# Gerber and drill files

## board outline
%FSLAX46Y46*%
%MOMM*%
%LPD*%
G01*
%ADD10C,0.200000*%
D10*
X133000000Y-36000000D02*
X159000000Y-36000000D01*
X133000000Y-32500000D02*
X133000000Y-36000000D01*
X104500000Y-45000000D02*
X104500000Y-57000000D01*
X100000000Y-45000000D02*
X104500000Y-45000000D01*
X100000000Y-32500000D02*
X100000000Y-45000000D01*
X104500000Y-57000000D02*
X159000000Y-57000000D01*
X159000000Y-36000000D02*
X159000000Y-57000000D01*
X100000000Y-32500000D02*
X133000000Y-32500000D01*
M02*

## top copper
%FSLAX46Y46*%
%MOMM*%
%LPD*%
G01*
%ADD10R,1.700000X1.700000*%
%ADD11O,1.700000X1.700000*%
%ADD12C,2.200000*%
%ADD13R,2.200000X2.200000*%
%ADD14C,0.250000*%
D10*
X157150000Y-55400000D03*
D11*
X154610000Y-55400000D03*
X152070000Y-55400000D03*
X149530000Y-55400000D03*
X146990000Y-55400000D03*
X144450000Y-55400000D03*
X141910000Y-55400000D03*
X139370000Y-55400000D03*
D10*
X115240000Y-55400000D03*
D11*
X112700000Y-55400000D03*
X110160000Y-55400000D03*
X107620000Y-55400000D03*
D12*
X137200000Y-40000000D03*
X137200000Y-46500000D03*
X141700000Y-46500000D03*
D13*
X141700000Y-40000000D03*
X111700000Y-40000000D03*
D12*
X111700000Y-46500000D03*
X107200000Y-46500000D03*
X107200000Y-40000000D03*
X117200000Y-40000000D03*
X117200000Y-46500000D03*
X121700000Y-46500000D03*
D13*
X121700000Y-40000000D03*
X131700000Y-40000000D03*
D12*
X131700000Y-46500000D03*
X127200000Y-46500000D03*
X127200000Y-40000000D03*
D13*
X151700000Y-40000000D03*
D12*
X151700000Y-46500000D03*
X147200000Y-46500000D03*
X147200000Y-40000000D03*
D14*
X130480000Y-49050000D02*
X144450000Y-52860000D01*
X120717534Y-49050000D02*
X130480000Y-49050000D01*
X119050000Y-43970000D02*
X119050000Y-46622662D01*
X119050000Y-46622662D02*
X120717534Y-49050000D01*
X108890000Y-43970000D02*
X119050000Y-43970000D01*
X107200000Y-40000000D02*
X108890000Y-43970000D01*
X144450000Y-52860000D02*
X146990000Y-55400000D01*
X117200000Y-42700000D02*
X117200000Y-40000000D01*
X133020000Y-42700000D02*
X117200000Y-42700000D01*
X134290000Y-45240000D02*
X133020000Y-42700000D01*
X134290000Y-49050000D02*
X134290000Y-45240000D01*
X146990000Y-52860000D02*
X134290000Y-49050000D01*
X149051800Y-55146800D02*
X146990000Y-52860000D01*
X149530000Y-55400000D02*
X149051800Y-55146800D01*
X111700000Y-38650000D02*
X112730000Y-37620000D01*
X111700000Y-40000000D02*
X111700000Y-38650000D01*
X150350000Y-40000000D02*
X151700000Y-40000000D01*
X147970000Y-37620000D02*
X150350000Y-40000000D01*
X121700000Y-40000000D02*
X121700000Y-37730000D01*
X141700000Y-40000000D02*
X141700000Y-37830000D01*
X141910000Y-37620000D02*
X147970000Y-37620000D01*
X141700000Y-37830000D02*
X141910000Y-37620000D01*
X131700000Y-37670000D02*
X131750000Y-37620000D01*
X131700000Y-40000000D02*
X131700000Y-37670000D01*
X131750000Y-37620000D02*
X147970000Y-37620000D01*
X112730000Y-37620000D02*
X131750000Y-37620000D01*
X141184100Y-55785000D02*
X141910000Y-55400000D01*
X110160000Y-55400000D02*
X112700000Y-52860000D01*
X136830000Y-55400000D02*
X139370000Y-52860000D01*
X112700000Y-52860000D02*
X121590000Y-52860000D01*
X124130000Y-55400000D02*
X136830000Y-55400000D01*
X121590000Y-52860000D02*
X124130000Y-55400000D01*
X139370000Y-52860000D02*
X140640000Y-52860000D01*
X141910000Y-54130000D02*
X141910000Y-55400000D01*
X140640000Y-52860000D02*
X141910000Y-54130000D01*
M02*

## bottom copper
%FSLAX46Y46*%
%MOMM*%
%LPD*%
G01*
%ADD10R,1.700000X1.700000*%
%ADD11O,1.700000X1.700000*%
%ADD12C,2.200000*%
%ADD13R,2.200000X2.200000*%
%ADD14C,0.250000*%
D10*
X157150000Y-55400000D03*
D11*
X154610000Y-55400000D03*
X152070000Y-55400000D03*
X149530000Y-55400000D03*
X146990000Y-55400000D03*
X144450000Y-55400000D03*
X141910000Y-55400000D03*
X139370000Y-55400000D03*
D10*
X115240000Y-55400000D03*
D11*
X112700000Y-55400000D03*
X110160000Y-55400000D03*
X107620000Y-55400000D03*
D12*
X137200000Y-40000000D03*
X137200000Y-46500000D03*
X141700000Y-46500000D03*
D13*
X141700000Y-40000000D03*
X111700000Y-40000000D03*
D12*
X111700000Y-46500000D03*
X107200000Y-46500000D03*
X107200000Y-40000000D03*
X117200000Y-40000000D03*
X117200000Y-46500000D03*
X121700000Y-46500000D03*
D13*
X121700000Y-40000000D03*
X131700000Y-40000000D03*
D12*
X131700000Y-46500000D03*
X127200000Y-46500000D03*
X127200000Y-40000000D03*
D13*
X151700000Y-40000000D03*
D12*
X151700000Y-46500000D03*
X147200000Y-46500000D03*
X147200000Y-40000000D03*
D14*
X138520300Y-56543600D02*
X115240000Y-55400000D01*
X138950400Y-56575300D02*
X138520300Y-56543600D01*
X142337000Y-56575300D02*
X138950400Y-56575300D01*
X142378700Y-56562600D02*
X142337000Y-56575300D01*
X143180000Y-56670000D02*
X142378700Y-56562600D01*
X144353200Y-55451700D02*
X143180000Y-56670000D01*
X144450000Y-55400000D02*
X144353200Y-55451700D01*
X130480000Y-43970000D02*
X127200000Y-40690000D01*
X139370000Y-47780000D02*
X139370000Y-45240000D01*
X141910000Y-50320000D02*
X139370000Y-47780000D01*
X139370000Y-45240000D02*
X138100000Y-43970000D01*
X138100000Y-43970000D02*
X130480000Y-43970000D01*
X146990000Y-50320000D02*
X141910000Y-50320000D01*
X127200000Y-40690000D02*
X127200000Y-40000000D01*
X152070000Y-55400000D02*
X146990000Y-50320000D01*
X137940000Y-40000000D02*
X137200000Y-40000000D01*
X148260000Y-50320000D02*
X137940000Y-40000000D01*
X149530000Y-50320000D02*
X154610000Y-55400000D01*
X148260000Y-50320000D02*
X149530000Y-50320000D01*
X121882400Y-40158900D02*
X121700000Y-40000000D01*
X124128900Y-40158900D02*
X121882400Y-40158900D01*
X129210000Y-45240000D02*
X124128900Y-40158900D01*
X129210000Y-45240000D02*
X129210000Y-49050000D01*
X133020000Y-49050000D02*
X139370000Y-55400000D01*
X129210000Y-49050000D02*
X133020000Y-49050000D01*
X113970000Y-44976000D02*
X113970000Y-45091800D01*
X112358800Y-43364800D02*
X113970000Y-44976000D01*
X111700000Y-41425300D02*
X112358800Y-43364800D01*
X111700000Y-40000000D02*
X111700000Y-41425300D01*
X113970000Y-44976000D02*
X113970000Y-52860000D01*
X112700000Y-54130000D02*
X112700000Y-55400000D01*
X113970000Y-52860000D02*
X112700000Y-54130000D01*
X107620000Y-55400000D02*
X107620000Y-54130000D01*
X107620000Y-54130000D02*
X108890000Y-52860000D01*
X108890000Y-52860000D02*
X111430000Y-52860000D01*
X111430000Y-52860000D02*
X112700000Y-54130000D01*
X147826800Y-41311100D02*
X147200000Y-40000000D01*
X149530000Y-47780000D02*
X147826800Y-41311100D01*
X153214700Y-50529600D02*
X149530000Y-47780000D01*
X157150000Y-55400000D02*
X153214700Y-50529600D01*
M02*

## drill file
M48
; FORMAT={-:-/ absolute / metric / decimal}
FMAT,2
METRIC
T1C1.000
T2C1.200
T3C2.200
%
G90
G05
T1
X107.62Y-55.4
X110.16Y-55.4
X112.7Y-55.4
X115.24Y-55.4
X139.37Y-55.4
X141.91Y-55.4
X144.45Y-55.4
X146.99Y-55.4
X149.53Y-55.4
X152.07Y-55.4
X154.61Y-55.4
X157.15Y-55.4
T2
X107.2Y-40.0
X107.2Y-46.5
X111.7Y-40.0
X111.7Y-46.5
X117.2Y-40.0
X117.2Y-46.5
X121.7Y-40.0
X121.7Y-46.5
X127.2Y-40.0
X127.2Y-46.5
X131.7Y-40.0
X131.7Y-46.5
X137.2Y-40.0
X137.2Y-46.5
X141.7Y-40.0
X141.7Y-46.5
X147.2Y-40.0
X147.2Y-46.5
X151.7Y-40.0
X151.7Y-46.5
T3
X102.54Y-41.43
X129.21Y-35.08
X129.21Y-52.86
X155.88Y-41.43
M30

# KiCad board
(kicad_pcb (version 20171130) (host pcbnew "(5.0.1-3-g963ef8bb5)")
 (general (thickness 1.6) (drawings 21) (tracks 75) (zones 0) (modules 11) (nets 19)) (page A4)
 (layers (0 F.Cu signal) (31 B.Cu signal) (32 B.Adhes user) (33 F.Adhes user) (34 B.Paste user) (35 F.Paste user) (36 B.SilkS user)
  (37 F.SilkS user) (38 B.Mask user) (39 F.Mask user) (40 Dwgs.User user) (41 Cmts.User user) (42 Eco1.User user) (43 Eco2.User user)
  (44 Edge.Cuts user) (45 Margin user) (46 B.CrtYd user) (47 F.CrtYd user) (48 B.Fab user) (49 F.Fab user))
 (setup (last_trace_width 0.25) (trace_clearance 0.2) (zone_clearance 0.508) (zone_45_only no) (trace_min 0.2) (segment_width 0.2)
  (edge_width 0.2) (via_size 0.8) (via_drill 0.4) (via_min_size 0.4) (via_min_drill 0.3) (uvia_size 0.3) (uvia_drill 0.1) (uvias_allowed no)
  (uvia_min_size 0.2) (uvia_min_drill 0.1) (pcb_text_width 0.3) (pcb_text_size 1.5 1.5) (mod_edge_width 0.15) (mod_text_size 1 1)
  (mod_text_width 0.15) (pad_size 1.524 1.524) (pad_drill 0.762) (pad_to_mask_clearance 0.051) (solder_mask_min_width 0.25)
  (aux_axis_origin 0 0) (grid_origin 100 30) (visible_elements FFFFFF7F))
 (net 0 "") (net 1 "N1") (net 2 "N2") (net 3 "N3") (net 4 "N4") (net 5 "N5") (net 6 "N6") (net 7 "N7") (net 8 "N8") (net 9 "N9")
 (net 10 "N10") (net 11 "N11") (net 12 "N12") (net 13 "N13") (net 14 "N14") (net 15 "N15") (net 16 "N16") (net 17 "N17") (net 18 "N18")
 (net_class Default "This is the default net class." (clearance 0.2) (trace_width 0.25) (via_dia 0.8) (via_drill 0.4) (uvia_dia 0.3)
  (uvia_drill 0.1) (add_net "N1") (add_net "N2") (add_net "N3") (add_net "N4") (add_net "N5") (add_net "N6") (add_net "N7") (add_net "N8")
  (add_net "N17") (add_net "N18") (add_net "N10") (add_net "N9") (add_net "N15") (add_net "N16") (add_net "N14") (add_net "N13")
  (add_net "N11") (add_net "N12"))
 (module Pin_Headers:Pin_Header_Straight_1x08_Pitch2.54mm (layer F.Cu) (at 157.15 55.4 270)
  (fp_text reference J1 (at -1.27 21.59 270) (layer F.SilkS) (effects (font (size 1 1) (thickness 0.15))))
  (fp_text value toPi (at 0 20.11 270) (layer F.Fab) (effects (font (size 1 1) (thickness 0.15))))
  (pad 1 thru_hole rect (at 0 0 270) (size 1.7 1.7) (drill 1) (layers *.Cu *.Mask) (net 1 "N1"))
  (pad 2 thru_hole oval (at 0 2.54 270) (size 1.7 1.7) (drill 1) (layers *.Cu *.Mask) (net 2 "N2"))
  (pad 3 thru_hole oval (at 0 5.08 270) (size 1.7 1.7) (drill 1) (layers *.Cu *.Mask) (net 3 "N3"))
  (pad 4 thru_hole oval (at 0 7.62 270) (size 1.7 1.7) (drill 1) (layers *.Cu *.Mask) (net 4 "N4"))
  (pad 5 thru_hole oval (at 0 10.16 270) (size 1.7 1.7) (drill 1) (layers *.Cu *.Mask) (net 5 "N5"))
  (pad 6 thru_hole oval (at 0 12.7 270) (size 1.7 1.7) (drill 1) (layers *.Cu *.Mask) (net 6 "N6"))
  (pad 7 thru_hole oval (at 0 15.24 270) (size 1.7 1.7) (drill 1) (layers *.Cu *.Mask) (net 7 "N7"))
  (pad 8 thru_hole oval (at 0 17.78 270) (size 1.7 1.7) (drill 1) (layers *.Cu *.Mask) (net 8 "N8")))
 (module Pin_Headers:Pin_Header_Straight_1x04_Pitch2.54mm (layer F.Cu) (at 115.24 55.4 270)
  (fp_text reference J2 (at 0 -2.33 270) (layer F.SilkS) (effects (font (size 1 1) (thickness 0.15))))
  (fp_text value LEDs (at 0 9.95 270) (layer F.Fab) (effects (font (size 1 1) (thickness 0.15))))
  (pad 1 thru_hole rect (at 0 0 270) (size 1.7 1.7) (drill 1) (layers *.Cu *.Mask) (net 6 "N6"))
  (pad 2 thru_hole oval (at 0 2.54 270) (size 1.7 1.7) (drill 1) (layers *.Cu *.Mask) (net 8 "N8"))
  (pad 3 thru_hole oval (at 0 5.08 270) (size 1.7 1.7) (drill 1) (layers *.Cu *.Mask) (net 7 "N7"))
  (pad 4 thru_hole oval (at 0 7.62 270) (size 1.7 1.7) (drill 1) (layers *.Cu *.Mask) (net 8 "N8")))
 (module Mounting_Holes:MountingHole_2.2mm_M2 (layer F.Cu) (at 155.88 41.43)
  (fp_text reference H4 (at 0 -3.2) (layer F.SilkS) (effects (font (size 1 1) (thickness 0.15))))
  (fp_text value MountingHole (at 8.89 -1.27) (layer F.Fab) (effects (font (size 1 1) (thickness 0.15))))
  (pad 1 np_thru_hole circle (at 0 0) (size 2.2 2.2) (drill 2.2) (layers *.Cu *.Mask)))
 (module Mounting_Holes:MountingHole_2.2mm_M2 (layer F.Cu) (at 129.21 35.08)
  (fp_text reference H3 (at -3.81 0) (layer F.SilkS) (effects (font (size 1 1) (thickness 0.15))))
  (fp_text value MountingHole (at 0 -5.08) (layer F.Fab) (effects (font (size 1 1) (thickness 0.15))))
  (pad 1 np_thru_hole circle (at 0 0) (size 2.2 2.2) (drill 2.2) (layers *.Cu *.Mask)))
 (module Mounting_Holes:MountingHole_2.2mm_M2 (layer F.Cu) (at 102.54 41.43)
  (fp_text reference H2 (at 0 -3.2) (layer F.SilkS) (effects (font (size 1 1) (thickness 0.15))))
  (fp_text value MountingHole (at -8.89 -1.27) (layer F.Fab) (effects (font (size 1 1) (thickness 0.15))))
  (pad 1 np_thru_hole circle (at 0 0) (size 2.2 2.2) (drill 2.2) (layers *.Cu *.Mask)))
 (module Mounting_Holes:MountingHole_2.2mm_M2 (layer F.Cu) (at 129.21 52.86)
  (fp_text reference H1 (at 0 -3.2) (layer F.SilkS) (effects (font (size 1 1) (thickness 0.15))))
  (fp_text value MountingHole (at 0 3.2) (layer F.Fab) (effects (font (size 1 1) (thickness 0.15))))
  (pad 1 np_thru_hole circle (at 0 0) (size 2.2 2.2) (drill 2.2) (layers *.Cu *.Mask)))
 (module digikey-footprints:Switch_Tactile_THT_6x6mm (layer F.Cu) (at 141.7 40 270)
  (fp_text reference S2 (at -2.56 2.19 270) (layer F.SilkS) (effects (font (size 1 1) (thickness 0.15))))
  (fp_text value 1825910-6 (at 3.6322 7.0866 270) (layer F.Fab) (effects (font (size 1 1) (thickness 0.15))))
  (pad 3 thru_hole circle (at 0 4.5 270) (size 2.2 2.2) (drill 1.2) (layers *.Cu *.Mask) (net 2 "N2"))
  (pad 4 thru_hole circle (at 6.5 4.5 270) (size 2.2 2.2) (drill 1.2) (layers *.Cu *.Mask) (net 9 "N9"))
  (pad 2 thru_hole circle (at 6.5 0 270) (size 2.2 2.2) (drill 1.2) (layers *.Cu *.Mask) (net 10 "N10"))
  (pad 1 thru_hole rect (at 0 0 270) (size 2.2 2.2) (drill 1.2) (layers *.Cu *.Mask) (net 8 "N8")))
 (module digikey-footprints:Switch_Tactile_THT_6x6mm (layer F.Cu) (at 111.7 40 270)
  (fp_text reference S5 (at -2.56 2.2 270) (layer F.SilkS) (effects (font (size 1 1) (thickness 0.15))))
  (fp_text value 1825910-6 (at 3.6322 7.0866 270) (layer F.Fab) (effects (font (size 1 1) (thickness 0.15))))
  (pad 1 thru_hole rect (at 0 0 270) (size 2.2 2.2) (drill 1.2) (layers *.Cu *.Mask) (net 8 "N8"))
  (pad 2 thru_hole circle (at 6.5 0 270) (size 2.2 2.2) (drill 1.2) (layers *.Cu *.Mask) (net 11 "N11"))
  (pad 4 thru_hole circle (at 6.5 4.5 270) (size 2.2 2.2) (drill 1.2) (layers *.Cu *.Mask) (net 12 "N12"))
  (pad 3 thru_hole circle (at 0 4.5 270) (size 2.2 2.2) (drill 1.2) (layers *.Cu *.Mask) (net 5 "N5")))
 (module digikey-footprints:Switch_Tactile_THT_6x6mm (layer F.Cu) (at 121.7 40 270)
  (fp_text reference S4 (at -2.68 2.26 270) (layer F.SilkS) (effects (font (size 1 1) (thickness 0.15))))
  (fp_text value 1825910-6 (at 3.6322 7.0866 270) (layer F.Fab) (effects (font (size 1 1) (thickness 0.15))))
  (pad 3 thru_hole circle (at 0 4.5 270) (size 2.2 2.2) (drill 1.2) (layers *.Cu *.Mask) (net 4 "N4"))
  (pad 4 thru_hole circle (at 6.5 4.5 270) (size 2.2 2.2) (drill 1.2) (layers *.Cu *.Mask) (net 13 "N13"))
  (pad 2 thru_hole circle (at 6.5 0 270) (size 2.2 2.2) (drill 1.2) (layers *.Cu *.Mask) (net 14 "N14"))
  (pad 1 thru_hole rect (at 0 0 270) (size 2.2 2.2) (drill 1.2) (layers *.Cu *.Mask) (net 8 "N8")))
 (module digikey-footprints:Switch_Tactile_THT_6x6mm (layer F.Cu) (at 131.7 40 270)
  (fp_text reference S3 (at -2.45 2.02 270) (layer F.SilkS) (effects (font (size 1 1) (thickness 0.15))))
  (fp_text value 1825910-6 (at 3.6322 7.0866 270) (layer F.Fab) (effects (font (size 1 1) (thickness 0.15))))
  (pad 1 thru_hole rect (at 0 0 270) (size 2.2 2.2) (drill 1.2) (layers *.Cu *.Mask) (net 8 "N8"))
  (pad 2 thru_hole circle (at 6.5 0 270) (size 2.2 2.2) (drill 1.2) (layers *.Cu *.Mask) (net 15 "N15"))
  (pad 4 thru_hole circle (at 6.5 4.5 270) (size 2.2 2.2) (drill 1.2) (layers *.Cu *.Mask) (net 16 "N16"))
  (pad 3 thru_hole circle (at 0 4.5 270) (size 2.2 2.2) (drill 1.2) (layers *.Cu *.Mask) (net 3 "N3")))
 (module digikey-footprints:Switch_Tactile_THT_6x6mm (layer F.Cu) (at 151.7 40 270)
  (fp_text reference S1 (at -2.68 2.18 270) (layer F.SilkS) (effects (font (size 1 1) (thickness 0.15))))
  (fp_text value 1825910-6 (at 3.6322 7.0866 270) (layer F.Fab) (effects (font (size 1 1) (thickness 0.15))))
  (pad 1 thru_hole rect (at 0 0 270) (size 2.2 2.2) (drill 1.2) (layers *.Cu *.Mask) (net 8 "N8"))
  (pad 2 thru_hole circle (at 6.5 0 270) (size 2.2 2.2) (drill 1.2) (layers *.Cu *.Mask) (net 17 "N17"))
  (pad 4 thru_hole circle (at 6.5 4.5 270) (size 2.2 2.2) (drill 1.2) (layers *.Cu *.Mask) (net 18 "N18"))
  (pad 3 thru_hole circle (at 0 4.5 270) (size 2.2 2.2) (drill 1.2) (layers *.Cu *.Mask) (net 1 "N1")))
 (gr_line (start 133 36) (end 159 36) (layer Edge.Cuts) (width 0.2))
 (gr_line (start 133 32.5) (end 133 36) (layer Edge.Cuts) (width 0.2))
 (gr_line (start 104.5 45) (end 104.5 57) (layer Edge.Cuts) (width 0.2))
 (gr_line (start 100 45) (end 104.5 45) (layer Edge.Cuts) (width 0.2))
 (gr_line (start 100 32.5) (end 100 45) (layer Edge.Cuts) (width 0.2))
 (gr_line (start 104.5 57) (end 159 57) (layer Edge.Cuts) (width 0.2))
 (gr_line (start 159 36) (end 159 57) (layer Edge.Cuts) (width 0.2))
 (gr_line (start 100 32.5) (end 133 32.5) (layer Edge.Cuts) (width 0.2))
 (segment (start 138.5203 56.5436) (end 115.24 55.4) (width 0.25) (layer B.Cu) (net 6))
 (segment (start 138.9504 56.5753) (end 138.5203 56.5436) (width 0.25) (layer B.Cu) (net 6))
 (segment (start 142.337 56.5753) (end 138.9504 56.5753) (width 0.25) (layer B.Cu) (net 6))
 (segment (start 142.3787 56.5626) (end 142.337 56.5753) (width 0.25) (layer B.Cu) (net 6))
 (segment (start 143.18 56.67) (end 142.3787 56.5626) (width 0.25) (layer B.Cu) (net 6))
 (segment (start 144.3532 55.4517) (end 143.18 56.67) (width 0.25) (layer B.Cu) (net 6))
 (segment (start 144.45 55.4) (end 144.3532 55.4517) (width 0.25) (layer B.Cu) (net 6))
 (segment (start 130.48 49.05) (end 144.45 52.86) (width 0.25) (layer F.Cu) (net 5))
 (segment (start 120.717534 49.05) (end 130.48 49.05) (width 0.25) (layer F.Cu) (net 5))
 (segment (start 119.05 43.97) (end 119.05 46.622662) (width 0.25) (layer F.Cu) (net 5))
 (segment (start 119.05 46.622662) (end 120.717534 49.05) (width 0.25) (layer F.Cu) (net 5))
 (segment (start 108.89 43.97) (end 119.05 43.97) (width 0.25) (layer F.Cu) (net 5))
 (segment (start 107.2 40) (end 108.89 43.97) (width 0.25) (layer F.Cu) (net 5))
 (segment (start 144.45 52.86) (end 146.99 55.4) (width 0.25) (layer F.Cu) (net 5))
 (segment (start 117.2 42.7) (end 117.2 40) (width 0.25) (layer F.Cu) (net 4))
 (segment (start 133.02 42.7) (end 117.2 42.7) (width 0.25) (layer F.Cu) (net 4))
 (segment (start 134.29 45.24) (end 133.02 42.7) (width 0.25) (layer F.Cu) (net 4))
 (segment (start 134.29 49.05) (end 134.29 45.24) (width 0.25) (layer F.Cu) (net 4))
 (segment (start 146.99 52.86) (end 134.29 49.05) (width 0.25) (layer F.Cu) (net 4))
 (segment (start 149.0518 55.1468) (end 146.99 52.86) (width 0.25) (layer F.Cu) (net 4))
 (segment (start 149.53 55.4) (end 149.0518 55.1468) (width 0.25) (layer F.Cu) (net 4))
 (segment (start 130.48 43.97) (end 127.2 40.69) (width 0.25) (layer B.Cu) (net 3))
 (segment (start 139.37 47.78) (end 139.37 45.24) (width 0.25) (layer B.Cu) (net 3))
 (segment (start 141.91 50.32) (end 139.37 47.78) (width 0.25) (layer B.Cu) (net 3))
 (segment (start 139.37 45.24) (end 138.1 43.97) (width 0.25) (layer B.Cu) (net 3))
 (segment (start 138.1 43.97) (end 130.48 43.97) (width 0.25) (layer B.Cu) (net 3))
 (segment (start 146.99 50.32) (end 141.91 50.32) (width 0.25) (layer B.Cu) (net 3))
 (segment (start 127.2 40.69) (end 127.2 40) (width 0.25) (layer B.Cu) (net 3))
 (segment (start 152.07 55.4) (end 146.99 50.32) (width 0.25) (layer B.Cu) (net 3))
 (segment (start 137.94 40) (end 137.2 40) (width 0.25) (layer B.Cu) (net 2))
 (segment (start 148.26 50.32) (end 137.94 40) (width 0.25) (layer B.Cu) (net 2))
 (segment (start 149.53 50.32) (end 154.61 55.4) (width 0.25) (layer B.Cu) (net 2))
 (segment (start 148.26 50.32) (end 149.53 50.32) (width 0.25) (layer B.Cu) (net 2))
 (segment (start 111.7 38.65) (end 112.73 37.62) (width 0.25) (layer F.Cu) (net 8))
 (segment (start 111.7 40) (end 111.7 38.65) (width 0.25) (layer F.Cu) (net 8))
 (segment (start 150.35 40) (end 151.7 40) (width 0.25) (layer F.Cu) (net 8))
 (segment (start 147.97 37.62) (end 150.35 40) (width 0.25) (layer F.Cu) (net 8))
 (segment (start 121.7 40) (end 121.7 37.73) (width 0.25) (layer F.Cu) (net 8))
 (segment (start 141.7 40) (end 141.7 37.83) (width 0.25) (layer F.Cu) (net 8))
 (segment (start 141.91 37.62) (end 147.97 37.62) (width 0.25) (layer F.Cu) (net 8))
 (segment (start 141.7 37.83) (end 141.91 37.62) (width 0.25) (layer F.Cu) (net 8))
 (segment (start 131.7 37.67) (end 131.75 37.62) (width 0.25) (layer F.Cu) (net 8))
 (segment (start 131.7 40) (end 131.7 37.67) (width 0.25) (layer F.Cu) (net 8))
 (segment (start 131.75 37.62) (end 147.97 37.62) (width 0.25) (layer F.Cu) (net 8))
 (segment (start 112.73 37.62) (end 131.75 37.62) (width 0.25) (layer F.Cu) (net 8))
 (segment (start 121.8824 40.1589) (end 121.7 40) (width 0.25) (layer B.Cu) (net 8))
 (segment (start 124.1289 40.1589) (end 121.8824 40.1589) (width 0.25) (layer B.Cu) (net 8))
 (segment (start 129.21 45.24) (end 124.1289 40.1589) (width 0.25) (layer B.Cu) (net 8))
 (segment (start 129.21 45.24) (end 129.21 49.05) (width 0.25) (layer B.Cu) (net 8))
 (segment (start 133.02 49.05) (end 139.37 55.4) (width 0.25) (layer B.Cu) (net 8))
 (segment (start 129.21 49.05) (end 133.02 49.05) (width 0.25) (layer B.Cu) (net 8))
 (segment (start 113.97 44.976) (end 113.97 45.0918) (width 0.25) (layer B.Cu) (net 8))
 (segment (start 112.3588 43.3648) (end 113.97 44.976) (width 0.25) (layer B.Cu) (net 8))
 (segment (start 111.7 41.4253) (end 112.3588 43.3648) (width 0.25) (layer B.Cu) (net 8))
 (segment (start 111.7 40) (end 111.7 41.4253) (width 0.25) (layer B.Cu) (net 8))
 (segment (start 113.97 44.976) (end 113.97 52.86) (width 0.25) (layer B.Cu) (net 8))
 (segment (start 112.7 54.13) (end 112.7 55.4) (width 0.25) (layer B.Cu) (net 8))
 (segment (start 113.97 52.86) (end 112.7 54.13) (width 0.25) (layer B.Cu) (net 8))
 (segment (start 107.62 55.4) (end 107.62 54.13) (width 0.25) (layer B.Cu) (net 8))
 (segment (start 107.62 54.13) (end 108.89 52.86) (width 0.25) (layer B.Cu) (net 8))
 (segment (start 108.89 52.86) (end 111.43 52.86) (width 0.25) (layer B.Cu) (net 8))
 (segment (start 111.43 52.86) (end 112.7 54.13) (width 0.25) (layer B.Cu) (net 8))
 (segment (start 141.1841 55.785) (end 141.91 55.4) (width 0.25) (layer F.Cu) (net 7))
 (segment (start 110.16 55.4) (end 112.7 52.86) (width 0.25) (layer F.Cu) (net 7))
 (segment (start 136.83 55.4) (end 139.37 52.86) (width 0.25) (layer F.Cu) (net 7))
 (segment (start 112.7 52.86) (end 121.59 52.86) (width 0.25) (layer F.Cu) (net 7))
 (segment (start 124.13 55.4) (end 136.83 55.4) (width 0.25) (layer F.Cu) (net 7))
 (segment (start 121.59 52.86) (end 124.13 55.4) (width 0.25) (layer F.Cu) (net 7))
 (segment (start 139.37 52.86) (end 140.64 52.86) (width 0.25) (layer F.Cu) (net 7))
 (segment (start 141.91 54.13) (end 141.91 55.4) (width 0.25) (layer F.Cu) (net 7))
 (segment (start 140.64 52.86) (end 141.91 54.13) (width 0.25) (layer F.Cu) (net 7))
 (segment (start 147.8268 41.3111) (end 147.2 40) (width 0.25) (layer B.Cu) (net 1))
 (segment (start 149.53 47.78) (end 147.8268 41.3111) (width 0.25) (layer B.Cu) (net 1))
 (segment (start 153.2147 50.5296) (end 149.53 47.78) (width 0.25) (layer B.Cu) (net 1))
 (segment (start 157.15 55.4) (end 153.2147 50.5296) (width 0.25) (layer B.Cu) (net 1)))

